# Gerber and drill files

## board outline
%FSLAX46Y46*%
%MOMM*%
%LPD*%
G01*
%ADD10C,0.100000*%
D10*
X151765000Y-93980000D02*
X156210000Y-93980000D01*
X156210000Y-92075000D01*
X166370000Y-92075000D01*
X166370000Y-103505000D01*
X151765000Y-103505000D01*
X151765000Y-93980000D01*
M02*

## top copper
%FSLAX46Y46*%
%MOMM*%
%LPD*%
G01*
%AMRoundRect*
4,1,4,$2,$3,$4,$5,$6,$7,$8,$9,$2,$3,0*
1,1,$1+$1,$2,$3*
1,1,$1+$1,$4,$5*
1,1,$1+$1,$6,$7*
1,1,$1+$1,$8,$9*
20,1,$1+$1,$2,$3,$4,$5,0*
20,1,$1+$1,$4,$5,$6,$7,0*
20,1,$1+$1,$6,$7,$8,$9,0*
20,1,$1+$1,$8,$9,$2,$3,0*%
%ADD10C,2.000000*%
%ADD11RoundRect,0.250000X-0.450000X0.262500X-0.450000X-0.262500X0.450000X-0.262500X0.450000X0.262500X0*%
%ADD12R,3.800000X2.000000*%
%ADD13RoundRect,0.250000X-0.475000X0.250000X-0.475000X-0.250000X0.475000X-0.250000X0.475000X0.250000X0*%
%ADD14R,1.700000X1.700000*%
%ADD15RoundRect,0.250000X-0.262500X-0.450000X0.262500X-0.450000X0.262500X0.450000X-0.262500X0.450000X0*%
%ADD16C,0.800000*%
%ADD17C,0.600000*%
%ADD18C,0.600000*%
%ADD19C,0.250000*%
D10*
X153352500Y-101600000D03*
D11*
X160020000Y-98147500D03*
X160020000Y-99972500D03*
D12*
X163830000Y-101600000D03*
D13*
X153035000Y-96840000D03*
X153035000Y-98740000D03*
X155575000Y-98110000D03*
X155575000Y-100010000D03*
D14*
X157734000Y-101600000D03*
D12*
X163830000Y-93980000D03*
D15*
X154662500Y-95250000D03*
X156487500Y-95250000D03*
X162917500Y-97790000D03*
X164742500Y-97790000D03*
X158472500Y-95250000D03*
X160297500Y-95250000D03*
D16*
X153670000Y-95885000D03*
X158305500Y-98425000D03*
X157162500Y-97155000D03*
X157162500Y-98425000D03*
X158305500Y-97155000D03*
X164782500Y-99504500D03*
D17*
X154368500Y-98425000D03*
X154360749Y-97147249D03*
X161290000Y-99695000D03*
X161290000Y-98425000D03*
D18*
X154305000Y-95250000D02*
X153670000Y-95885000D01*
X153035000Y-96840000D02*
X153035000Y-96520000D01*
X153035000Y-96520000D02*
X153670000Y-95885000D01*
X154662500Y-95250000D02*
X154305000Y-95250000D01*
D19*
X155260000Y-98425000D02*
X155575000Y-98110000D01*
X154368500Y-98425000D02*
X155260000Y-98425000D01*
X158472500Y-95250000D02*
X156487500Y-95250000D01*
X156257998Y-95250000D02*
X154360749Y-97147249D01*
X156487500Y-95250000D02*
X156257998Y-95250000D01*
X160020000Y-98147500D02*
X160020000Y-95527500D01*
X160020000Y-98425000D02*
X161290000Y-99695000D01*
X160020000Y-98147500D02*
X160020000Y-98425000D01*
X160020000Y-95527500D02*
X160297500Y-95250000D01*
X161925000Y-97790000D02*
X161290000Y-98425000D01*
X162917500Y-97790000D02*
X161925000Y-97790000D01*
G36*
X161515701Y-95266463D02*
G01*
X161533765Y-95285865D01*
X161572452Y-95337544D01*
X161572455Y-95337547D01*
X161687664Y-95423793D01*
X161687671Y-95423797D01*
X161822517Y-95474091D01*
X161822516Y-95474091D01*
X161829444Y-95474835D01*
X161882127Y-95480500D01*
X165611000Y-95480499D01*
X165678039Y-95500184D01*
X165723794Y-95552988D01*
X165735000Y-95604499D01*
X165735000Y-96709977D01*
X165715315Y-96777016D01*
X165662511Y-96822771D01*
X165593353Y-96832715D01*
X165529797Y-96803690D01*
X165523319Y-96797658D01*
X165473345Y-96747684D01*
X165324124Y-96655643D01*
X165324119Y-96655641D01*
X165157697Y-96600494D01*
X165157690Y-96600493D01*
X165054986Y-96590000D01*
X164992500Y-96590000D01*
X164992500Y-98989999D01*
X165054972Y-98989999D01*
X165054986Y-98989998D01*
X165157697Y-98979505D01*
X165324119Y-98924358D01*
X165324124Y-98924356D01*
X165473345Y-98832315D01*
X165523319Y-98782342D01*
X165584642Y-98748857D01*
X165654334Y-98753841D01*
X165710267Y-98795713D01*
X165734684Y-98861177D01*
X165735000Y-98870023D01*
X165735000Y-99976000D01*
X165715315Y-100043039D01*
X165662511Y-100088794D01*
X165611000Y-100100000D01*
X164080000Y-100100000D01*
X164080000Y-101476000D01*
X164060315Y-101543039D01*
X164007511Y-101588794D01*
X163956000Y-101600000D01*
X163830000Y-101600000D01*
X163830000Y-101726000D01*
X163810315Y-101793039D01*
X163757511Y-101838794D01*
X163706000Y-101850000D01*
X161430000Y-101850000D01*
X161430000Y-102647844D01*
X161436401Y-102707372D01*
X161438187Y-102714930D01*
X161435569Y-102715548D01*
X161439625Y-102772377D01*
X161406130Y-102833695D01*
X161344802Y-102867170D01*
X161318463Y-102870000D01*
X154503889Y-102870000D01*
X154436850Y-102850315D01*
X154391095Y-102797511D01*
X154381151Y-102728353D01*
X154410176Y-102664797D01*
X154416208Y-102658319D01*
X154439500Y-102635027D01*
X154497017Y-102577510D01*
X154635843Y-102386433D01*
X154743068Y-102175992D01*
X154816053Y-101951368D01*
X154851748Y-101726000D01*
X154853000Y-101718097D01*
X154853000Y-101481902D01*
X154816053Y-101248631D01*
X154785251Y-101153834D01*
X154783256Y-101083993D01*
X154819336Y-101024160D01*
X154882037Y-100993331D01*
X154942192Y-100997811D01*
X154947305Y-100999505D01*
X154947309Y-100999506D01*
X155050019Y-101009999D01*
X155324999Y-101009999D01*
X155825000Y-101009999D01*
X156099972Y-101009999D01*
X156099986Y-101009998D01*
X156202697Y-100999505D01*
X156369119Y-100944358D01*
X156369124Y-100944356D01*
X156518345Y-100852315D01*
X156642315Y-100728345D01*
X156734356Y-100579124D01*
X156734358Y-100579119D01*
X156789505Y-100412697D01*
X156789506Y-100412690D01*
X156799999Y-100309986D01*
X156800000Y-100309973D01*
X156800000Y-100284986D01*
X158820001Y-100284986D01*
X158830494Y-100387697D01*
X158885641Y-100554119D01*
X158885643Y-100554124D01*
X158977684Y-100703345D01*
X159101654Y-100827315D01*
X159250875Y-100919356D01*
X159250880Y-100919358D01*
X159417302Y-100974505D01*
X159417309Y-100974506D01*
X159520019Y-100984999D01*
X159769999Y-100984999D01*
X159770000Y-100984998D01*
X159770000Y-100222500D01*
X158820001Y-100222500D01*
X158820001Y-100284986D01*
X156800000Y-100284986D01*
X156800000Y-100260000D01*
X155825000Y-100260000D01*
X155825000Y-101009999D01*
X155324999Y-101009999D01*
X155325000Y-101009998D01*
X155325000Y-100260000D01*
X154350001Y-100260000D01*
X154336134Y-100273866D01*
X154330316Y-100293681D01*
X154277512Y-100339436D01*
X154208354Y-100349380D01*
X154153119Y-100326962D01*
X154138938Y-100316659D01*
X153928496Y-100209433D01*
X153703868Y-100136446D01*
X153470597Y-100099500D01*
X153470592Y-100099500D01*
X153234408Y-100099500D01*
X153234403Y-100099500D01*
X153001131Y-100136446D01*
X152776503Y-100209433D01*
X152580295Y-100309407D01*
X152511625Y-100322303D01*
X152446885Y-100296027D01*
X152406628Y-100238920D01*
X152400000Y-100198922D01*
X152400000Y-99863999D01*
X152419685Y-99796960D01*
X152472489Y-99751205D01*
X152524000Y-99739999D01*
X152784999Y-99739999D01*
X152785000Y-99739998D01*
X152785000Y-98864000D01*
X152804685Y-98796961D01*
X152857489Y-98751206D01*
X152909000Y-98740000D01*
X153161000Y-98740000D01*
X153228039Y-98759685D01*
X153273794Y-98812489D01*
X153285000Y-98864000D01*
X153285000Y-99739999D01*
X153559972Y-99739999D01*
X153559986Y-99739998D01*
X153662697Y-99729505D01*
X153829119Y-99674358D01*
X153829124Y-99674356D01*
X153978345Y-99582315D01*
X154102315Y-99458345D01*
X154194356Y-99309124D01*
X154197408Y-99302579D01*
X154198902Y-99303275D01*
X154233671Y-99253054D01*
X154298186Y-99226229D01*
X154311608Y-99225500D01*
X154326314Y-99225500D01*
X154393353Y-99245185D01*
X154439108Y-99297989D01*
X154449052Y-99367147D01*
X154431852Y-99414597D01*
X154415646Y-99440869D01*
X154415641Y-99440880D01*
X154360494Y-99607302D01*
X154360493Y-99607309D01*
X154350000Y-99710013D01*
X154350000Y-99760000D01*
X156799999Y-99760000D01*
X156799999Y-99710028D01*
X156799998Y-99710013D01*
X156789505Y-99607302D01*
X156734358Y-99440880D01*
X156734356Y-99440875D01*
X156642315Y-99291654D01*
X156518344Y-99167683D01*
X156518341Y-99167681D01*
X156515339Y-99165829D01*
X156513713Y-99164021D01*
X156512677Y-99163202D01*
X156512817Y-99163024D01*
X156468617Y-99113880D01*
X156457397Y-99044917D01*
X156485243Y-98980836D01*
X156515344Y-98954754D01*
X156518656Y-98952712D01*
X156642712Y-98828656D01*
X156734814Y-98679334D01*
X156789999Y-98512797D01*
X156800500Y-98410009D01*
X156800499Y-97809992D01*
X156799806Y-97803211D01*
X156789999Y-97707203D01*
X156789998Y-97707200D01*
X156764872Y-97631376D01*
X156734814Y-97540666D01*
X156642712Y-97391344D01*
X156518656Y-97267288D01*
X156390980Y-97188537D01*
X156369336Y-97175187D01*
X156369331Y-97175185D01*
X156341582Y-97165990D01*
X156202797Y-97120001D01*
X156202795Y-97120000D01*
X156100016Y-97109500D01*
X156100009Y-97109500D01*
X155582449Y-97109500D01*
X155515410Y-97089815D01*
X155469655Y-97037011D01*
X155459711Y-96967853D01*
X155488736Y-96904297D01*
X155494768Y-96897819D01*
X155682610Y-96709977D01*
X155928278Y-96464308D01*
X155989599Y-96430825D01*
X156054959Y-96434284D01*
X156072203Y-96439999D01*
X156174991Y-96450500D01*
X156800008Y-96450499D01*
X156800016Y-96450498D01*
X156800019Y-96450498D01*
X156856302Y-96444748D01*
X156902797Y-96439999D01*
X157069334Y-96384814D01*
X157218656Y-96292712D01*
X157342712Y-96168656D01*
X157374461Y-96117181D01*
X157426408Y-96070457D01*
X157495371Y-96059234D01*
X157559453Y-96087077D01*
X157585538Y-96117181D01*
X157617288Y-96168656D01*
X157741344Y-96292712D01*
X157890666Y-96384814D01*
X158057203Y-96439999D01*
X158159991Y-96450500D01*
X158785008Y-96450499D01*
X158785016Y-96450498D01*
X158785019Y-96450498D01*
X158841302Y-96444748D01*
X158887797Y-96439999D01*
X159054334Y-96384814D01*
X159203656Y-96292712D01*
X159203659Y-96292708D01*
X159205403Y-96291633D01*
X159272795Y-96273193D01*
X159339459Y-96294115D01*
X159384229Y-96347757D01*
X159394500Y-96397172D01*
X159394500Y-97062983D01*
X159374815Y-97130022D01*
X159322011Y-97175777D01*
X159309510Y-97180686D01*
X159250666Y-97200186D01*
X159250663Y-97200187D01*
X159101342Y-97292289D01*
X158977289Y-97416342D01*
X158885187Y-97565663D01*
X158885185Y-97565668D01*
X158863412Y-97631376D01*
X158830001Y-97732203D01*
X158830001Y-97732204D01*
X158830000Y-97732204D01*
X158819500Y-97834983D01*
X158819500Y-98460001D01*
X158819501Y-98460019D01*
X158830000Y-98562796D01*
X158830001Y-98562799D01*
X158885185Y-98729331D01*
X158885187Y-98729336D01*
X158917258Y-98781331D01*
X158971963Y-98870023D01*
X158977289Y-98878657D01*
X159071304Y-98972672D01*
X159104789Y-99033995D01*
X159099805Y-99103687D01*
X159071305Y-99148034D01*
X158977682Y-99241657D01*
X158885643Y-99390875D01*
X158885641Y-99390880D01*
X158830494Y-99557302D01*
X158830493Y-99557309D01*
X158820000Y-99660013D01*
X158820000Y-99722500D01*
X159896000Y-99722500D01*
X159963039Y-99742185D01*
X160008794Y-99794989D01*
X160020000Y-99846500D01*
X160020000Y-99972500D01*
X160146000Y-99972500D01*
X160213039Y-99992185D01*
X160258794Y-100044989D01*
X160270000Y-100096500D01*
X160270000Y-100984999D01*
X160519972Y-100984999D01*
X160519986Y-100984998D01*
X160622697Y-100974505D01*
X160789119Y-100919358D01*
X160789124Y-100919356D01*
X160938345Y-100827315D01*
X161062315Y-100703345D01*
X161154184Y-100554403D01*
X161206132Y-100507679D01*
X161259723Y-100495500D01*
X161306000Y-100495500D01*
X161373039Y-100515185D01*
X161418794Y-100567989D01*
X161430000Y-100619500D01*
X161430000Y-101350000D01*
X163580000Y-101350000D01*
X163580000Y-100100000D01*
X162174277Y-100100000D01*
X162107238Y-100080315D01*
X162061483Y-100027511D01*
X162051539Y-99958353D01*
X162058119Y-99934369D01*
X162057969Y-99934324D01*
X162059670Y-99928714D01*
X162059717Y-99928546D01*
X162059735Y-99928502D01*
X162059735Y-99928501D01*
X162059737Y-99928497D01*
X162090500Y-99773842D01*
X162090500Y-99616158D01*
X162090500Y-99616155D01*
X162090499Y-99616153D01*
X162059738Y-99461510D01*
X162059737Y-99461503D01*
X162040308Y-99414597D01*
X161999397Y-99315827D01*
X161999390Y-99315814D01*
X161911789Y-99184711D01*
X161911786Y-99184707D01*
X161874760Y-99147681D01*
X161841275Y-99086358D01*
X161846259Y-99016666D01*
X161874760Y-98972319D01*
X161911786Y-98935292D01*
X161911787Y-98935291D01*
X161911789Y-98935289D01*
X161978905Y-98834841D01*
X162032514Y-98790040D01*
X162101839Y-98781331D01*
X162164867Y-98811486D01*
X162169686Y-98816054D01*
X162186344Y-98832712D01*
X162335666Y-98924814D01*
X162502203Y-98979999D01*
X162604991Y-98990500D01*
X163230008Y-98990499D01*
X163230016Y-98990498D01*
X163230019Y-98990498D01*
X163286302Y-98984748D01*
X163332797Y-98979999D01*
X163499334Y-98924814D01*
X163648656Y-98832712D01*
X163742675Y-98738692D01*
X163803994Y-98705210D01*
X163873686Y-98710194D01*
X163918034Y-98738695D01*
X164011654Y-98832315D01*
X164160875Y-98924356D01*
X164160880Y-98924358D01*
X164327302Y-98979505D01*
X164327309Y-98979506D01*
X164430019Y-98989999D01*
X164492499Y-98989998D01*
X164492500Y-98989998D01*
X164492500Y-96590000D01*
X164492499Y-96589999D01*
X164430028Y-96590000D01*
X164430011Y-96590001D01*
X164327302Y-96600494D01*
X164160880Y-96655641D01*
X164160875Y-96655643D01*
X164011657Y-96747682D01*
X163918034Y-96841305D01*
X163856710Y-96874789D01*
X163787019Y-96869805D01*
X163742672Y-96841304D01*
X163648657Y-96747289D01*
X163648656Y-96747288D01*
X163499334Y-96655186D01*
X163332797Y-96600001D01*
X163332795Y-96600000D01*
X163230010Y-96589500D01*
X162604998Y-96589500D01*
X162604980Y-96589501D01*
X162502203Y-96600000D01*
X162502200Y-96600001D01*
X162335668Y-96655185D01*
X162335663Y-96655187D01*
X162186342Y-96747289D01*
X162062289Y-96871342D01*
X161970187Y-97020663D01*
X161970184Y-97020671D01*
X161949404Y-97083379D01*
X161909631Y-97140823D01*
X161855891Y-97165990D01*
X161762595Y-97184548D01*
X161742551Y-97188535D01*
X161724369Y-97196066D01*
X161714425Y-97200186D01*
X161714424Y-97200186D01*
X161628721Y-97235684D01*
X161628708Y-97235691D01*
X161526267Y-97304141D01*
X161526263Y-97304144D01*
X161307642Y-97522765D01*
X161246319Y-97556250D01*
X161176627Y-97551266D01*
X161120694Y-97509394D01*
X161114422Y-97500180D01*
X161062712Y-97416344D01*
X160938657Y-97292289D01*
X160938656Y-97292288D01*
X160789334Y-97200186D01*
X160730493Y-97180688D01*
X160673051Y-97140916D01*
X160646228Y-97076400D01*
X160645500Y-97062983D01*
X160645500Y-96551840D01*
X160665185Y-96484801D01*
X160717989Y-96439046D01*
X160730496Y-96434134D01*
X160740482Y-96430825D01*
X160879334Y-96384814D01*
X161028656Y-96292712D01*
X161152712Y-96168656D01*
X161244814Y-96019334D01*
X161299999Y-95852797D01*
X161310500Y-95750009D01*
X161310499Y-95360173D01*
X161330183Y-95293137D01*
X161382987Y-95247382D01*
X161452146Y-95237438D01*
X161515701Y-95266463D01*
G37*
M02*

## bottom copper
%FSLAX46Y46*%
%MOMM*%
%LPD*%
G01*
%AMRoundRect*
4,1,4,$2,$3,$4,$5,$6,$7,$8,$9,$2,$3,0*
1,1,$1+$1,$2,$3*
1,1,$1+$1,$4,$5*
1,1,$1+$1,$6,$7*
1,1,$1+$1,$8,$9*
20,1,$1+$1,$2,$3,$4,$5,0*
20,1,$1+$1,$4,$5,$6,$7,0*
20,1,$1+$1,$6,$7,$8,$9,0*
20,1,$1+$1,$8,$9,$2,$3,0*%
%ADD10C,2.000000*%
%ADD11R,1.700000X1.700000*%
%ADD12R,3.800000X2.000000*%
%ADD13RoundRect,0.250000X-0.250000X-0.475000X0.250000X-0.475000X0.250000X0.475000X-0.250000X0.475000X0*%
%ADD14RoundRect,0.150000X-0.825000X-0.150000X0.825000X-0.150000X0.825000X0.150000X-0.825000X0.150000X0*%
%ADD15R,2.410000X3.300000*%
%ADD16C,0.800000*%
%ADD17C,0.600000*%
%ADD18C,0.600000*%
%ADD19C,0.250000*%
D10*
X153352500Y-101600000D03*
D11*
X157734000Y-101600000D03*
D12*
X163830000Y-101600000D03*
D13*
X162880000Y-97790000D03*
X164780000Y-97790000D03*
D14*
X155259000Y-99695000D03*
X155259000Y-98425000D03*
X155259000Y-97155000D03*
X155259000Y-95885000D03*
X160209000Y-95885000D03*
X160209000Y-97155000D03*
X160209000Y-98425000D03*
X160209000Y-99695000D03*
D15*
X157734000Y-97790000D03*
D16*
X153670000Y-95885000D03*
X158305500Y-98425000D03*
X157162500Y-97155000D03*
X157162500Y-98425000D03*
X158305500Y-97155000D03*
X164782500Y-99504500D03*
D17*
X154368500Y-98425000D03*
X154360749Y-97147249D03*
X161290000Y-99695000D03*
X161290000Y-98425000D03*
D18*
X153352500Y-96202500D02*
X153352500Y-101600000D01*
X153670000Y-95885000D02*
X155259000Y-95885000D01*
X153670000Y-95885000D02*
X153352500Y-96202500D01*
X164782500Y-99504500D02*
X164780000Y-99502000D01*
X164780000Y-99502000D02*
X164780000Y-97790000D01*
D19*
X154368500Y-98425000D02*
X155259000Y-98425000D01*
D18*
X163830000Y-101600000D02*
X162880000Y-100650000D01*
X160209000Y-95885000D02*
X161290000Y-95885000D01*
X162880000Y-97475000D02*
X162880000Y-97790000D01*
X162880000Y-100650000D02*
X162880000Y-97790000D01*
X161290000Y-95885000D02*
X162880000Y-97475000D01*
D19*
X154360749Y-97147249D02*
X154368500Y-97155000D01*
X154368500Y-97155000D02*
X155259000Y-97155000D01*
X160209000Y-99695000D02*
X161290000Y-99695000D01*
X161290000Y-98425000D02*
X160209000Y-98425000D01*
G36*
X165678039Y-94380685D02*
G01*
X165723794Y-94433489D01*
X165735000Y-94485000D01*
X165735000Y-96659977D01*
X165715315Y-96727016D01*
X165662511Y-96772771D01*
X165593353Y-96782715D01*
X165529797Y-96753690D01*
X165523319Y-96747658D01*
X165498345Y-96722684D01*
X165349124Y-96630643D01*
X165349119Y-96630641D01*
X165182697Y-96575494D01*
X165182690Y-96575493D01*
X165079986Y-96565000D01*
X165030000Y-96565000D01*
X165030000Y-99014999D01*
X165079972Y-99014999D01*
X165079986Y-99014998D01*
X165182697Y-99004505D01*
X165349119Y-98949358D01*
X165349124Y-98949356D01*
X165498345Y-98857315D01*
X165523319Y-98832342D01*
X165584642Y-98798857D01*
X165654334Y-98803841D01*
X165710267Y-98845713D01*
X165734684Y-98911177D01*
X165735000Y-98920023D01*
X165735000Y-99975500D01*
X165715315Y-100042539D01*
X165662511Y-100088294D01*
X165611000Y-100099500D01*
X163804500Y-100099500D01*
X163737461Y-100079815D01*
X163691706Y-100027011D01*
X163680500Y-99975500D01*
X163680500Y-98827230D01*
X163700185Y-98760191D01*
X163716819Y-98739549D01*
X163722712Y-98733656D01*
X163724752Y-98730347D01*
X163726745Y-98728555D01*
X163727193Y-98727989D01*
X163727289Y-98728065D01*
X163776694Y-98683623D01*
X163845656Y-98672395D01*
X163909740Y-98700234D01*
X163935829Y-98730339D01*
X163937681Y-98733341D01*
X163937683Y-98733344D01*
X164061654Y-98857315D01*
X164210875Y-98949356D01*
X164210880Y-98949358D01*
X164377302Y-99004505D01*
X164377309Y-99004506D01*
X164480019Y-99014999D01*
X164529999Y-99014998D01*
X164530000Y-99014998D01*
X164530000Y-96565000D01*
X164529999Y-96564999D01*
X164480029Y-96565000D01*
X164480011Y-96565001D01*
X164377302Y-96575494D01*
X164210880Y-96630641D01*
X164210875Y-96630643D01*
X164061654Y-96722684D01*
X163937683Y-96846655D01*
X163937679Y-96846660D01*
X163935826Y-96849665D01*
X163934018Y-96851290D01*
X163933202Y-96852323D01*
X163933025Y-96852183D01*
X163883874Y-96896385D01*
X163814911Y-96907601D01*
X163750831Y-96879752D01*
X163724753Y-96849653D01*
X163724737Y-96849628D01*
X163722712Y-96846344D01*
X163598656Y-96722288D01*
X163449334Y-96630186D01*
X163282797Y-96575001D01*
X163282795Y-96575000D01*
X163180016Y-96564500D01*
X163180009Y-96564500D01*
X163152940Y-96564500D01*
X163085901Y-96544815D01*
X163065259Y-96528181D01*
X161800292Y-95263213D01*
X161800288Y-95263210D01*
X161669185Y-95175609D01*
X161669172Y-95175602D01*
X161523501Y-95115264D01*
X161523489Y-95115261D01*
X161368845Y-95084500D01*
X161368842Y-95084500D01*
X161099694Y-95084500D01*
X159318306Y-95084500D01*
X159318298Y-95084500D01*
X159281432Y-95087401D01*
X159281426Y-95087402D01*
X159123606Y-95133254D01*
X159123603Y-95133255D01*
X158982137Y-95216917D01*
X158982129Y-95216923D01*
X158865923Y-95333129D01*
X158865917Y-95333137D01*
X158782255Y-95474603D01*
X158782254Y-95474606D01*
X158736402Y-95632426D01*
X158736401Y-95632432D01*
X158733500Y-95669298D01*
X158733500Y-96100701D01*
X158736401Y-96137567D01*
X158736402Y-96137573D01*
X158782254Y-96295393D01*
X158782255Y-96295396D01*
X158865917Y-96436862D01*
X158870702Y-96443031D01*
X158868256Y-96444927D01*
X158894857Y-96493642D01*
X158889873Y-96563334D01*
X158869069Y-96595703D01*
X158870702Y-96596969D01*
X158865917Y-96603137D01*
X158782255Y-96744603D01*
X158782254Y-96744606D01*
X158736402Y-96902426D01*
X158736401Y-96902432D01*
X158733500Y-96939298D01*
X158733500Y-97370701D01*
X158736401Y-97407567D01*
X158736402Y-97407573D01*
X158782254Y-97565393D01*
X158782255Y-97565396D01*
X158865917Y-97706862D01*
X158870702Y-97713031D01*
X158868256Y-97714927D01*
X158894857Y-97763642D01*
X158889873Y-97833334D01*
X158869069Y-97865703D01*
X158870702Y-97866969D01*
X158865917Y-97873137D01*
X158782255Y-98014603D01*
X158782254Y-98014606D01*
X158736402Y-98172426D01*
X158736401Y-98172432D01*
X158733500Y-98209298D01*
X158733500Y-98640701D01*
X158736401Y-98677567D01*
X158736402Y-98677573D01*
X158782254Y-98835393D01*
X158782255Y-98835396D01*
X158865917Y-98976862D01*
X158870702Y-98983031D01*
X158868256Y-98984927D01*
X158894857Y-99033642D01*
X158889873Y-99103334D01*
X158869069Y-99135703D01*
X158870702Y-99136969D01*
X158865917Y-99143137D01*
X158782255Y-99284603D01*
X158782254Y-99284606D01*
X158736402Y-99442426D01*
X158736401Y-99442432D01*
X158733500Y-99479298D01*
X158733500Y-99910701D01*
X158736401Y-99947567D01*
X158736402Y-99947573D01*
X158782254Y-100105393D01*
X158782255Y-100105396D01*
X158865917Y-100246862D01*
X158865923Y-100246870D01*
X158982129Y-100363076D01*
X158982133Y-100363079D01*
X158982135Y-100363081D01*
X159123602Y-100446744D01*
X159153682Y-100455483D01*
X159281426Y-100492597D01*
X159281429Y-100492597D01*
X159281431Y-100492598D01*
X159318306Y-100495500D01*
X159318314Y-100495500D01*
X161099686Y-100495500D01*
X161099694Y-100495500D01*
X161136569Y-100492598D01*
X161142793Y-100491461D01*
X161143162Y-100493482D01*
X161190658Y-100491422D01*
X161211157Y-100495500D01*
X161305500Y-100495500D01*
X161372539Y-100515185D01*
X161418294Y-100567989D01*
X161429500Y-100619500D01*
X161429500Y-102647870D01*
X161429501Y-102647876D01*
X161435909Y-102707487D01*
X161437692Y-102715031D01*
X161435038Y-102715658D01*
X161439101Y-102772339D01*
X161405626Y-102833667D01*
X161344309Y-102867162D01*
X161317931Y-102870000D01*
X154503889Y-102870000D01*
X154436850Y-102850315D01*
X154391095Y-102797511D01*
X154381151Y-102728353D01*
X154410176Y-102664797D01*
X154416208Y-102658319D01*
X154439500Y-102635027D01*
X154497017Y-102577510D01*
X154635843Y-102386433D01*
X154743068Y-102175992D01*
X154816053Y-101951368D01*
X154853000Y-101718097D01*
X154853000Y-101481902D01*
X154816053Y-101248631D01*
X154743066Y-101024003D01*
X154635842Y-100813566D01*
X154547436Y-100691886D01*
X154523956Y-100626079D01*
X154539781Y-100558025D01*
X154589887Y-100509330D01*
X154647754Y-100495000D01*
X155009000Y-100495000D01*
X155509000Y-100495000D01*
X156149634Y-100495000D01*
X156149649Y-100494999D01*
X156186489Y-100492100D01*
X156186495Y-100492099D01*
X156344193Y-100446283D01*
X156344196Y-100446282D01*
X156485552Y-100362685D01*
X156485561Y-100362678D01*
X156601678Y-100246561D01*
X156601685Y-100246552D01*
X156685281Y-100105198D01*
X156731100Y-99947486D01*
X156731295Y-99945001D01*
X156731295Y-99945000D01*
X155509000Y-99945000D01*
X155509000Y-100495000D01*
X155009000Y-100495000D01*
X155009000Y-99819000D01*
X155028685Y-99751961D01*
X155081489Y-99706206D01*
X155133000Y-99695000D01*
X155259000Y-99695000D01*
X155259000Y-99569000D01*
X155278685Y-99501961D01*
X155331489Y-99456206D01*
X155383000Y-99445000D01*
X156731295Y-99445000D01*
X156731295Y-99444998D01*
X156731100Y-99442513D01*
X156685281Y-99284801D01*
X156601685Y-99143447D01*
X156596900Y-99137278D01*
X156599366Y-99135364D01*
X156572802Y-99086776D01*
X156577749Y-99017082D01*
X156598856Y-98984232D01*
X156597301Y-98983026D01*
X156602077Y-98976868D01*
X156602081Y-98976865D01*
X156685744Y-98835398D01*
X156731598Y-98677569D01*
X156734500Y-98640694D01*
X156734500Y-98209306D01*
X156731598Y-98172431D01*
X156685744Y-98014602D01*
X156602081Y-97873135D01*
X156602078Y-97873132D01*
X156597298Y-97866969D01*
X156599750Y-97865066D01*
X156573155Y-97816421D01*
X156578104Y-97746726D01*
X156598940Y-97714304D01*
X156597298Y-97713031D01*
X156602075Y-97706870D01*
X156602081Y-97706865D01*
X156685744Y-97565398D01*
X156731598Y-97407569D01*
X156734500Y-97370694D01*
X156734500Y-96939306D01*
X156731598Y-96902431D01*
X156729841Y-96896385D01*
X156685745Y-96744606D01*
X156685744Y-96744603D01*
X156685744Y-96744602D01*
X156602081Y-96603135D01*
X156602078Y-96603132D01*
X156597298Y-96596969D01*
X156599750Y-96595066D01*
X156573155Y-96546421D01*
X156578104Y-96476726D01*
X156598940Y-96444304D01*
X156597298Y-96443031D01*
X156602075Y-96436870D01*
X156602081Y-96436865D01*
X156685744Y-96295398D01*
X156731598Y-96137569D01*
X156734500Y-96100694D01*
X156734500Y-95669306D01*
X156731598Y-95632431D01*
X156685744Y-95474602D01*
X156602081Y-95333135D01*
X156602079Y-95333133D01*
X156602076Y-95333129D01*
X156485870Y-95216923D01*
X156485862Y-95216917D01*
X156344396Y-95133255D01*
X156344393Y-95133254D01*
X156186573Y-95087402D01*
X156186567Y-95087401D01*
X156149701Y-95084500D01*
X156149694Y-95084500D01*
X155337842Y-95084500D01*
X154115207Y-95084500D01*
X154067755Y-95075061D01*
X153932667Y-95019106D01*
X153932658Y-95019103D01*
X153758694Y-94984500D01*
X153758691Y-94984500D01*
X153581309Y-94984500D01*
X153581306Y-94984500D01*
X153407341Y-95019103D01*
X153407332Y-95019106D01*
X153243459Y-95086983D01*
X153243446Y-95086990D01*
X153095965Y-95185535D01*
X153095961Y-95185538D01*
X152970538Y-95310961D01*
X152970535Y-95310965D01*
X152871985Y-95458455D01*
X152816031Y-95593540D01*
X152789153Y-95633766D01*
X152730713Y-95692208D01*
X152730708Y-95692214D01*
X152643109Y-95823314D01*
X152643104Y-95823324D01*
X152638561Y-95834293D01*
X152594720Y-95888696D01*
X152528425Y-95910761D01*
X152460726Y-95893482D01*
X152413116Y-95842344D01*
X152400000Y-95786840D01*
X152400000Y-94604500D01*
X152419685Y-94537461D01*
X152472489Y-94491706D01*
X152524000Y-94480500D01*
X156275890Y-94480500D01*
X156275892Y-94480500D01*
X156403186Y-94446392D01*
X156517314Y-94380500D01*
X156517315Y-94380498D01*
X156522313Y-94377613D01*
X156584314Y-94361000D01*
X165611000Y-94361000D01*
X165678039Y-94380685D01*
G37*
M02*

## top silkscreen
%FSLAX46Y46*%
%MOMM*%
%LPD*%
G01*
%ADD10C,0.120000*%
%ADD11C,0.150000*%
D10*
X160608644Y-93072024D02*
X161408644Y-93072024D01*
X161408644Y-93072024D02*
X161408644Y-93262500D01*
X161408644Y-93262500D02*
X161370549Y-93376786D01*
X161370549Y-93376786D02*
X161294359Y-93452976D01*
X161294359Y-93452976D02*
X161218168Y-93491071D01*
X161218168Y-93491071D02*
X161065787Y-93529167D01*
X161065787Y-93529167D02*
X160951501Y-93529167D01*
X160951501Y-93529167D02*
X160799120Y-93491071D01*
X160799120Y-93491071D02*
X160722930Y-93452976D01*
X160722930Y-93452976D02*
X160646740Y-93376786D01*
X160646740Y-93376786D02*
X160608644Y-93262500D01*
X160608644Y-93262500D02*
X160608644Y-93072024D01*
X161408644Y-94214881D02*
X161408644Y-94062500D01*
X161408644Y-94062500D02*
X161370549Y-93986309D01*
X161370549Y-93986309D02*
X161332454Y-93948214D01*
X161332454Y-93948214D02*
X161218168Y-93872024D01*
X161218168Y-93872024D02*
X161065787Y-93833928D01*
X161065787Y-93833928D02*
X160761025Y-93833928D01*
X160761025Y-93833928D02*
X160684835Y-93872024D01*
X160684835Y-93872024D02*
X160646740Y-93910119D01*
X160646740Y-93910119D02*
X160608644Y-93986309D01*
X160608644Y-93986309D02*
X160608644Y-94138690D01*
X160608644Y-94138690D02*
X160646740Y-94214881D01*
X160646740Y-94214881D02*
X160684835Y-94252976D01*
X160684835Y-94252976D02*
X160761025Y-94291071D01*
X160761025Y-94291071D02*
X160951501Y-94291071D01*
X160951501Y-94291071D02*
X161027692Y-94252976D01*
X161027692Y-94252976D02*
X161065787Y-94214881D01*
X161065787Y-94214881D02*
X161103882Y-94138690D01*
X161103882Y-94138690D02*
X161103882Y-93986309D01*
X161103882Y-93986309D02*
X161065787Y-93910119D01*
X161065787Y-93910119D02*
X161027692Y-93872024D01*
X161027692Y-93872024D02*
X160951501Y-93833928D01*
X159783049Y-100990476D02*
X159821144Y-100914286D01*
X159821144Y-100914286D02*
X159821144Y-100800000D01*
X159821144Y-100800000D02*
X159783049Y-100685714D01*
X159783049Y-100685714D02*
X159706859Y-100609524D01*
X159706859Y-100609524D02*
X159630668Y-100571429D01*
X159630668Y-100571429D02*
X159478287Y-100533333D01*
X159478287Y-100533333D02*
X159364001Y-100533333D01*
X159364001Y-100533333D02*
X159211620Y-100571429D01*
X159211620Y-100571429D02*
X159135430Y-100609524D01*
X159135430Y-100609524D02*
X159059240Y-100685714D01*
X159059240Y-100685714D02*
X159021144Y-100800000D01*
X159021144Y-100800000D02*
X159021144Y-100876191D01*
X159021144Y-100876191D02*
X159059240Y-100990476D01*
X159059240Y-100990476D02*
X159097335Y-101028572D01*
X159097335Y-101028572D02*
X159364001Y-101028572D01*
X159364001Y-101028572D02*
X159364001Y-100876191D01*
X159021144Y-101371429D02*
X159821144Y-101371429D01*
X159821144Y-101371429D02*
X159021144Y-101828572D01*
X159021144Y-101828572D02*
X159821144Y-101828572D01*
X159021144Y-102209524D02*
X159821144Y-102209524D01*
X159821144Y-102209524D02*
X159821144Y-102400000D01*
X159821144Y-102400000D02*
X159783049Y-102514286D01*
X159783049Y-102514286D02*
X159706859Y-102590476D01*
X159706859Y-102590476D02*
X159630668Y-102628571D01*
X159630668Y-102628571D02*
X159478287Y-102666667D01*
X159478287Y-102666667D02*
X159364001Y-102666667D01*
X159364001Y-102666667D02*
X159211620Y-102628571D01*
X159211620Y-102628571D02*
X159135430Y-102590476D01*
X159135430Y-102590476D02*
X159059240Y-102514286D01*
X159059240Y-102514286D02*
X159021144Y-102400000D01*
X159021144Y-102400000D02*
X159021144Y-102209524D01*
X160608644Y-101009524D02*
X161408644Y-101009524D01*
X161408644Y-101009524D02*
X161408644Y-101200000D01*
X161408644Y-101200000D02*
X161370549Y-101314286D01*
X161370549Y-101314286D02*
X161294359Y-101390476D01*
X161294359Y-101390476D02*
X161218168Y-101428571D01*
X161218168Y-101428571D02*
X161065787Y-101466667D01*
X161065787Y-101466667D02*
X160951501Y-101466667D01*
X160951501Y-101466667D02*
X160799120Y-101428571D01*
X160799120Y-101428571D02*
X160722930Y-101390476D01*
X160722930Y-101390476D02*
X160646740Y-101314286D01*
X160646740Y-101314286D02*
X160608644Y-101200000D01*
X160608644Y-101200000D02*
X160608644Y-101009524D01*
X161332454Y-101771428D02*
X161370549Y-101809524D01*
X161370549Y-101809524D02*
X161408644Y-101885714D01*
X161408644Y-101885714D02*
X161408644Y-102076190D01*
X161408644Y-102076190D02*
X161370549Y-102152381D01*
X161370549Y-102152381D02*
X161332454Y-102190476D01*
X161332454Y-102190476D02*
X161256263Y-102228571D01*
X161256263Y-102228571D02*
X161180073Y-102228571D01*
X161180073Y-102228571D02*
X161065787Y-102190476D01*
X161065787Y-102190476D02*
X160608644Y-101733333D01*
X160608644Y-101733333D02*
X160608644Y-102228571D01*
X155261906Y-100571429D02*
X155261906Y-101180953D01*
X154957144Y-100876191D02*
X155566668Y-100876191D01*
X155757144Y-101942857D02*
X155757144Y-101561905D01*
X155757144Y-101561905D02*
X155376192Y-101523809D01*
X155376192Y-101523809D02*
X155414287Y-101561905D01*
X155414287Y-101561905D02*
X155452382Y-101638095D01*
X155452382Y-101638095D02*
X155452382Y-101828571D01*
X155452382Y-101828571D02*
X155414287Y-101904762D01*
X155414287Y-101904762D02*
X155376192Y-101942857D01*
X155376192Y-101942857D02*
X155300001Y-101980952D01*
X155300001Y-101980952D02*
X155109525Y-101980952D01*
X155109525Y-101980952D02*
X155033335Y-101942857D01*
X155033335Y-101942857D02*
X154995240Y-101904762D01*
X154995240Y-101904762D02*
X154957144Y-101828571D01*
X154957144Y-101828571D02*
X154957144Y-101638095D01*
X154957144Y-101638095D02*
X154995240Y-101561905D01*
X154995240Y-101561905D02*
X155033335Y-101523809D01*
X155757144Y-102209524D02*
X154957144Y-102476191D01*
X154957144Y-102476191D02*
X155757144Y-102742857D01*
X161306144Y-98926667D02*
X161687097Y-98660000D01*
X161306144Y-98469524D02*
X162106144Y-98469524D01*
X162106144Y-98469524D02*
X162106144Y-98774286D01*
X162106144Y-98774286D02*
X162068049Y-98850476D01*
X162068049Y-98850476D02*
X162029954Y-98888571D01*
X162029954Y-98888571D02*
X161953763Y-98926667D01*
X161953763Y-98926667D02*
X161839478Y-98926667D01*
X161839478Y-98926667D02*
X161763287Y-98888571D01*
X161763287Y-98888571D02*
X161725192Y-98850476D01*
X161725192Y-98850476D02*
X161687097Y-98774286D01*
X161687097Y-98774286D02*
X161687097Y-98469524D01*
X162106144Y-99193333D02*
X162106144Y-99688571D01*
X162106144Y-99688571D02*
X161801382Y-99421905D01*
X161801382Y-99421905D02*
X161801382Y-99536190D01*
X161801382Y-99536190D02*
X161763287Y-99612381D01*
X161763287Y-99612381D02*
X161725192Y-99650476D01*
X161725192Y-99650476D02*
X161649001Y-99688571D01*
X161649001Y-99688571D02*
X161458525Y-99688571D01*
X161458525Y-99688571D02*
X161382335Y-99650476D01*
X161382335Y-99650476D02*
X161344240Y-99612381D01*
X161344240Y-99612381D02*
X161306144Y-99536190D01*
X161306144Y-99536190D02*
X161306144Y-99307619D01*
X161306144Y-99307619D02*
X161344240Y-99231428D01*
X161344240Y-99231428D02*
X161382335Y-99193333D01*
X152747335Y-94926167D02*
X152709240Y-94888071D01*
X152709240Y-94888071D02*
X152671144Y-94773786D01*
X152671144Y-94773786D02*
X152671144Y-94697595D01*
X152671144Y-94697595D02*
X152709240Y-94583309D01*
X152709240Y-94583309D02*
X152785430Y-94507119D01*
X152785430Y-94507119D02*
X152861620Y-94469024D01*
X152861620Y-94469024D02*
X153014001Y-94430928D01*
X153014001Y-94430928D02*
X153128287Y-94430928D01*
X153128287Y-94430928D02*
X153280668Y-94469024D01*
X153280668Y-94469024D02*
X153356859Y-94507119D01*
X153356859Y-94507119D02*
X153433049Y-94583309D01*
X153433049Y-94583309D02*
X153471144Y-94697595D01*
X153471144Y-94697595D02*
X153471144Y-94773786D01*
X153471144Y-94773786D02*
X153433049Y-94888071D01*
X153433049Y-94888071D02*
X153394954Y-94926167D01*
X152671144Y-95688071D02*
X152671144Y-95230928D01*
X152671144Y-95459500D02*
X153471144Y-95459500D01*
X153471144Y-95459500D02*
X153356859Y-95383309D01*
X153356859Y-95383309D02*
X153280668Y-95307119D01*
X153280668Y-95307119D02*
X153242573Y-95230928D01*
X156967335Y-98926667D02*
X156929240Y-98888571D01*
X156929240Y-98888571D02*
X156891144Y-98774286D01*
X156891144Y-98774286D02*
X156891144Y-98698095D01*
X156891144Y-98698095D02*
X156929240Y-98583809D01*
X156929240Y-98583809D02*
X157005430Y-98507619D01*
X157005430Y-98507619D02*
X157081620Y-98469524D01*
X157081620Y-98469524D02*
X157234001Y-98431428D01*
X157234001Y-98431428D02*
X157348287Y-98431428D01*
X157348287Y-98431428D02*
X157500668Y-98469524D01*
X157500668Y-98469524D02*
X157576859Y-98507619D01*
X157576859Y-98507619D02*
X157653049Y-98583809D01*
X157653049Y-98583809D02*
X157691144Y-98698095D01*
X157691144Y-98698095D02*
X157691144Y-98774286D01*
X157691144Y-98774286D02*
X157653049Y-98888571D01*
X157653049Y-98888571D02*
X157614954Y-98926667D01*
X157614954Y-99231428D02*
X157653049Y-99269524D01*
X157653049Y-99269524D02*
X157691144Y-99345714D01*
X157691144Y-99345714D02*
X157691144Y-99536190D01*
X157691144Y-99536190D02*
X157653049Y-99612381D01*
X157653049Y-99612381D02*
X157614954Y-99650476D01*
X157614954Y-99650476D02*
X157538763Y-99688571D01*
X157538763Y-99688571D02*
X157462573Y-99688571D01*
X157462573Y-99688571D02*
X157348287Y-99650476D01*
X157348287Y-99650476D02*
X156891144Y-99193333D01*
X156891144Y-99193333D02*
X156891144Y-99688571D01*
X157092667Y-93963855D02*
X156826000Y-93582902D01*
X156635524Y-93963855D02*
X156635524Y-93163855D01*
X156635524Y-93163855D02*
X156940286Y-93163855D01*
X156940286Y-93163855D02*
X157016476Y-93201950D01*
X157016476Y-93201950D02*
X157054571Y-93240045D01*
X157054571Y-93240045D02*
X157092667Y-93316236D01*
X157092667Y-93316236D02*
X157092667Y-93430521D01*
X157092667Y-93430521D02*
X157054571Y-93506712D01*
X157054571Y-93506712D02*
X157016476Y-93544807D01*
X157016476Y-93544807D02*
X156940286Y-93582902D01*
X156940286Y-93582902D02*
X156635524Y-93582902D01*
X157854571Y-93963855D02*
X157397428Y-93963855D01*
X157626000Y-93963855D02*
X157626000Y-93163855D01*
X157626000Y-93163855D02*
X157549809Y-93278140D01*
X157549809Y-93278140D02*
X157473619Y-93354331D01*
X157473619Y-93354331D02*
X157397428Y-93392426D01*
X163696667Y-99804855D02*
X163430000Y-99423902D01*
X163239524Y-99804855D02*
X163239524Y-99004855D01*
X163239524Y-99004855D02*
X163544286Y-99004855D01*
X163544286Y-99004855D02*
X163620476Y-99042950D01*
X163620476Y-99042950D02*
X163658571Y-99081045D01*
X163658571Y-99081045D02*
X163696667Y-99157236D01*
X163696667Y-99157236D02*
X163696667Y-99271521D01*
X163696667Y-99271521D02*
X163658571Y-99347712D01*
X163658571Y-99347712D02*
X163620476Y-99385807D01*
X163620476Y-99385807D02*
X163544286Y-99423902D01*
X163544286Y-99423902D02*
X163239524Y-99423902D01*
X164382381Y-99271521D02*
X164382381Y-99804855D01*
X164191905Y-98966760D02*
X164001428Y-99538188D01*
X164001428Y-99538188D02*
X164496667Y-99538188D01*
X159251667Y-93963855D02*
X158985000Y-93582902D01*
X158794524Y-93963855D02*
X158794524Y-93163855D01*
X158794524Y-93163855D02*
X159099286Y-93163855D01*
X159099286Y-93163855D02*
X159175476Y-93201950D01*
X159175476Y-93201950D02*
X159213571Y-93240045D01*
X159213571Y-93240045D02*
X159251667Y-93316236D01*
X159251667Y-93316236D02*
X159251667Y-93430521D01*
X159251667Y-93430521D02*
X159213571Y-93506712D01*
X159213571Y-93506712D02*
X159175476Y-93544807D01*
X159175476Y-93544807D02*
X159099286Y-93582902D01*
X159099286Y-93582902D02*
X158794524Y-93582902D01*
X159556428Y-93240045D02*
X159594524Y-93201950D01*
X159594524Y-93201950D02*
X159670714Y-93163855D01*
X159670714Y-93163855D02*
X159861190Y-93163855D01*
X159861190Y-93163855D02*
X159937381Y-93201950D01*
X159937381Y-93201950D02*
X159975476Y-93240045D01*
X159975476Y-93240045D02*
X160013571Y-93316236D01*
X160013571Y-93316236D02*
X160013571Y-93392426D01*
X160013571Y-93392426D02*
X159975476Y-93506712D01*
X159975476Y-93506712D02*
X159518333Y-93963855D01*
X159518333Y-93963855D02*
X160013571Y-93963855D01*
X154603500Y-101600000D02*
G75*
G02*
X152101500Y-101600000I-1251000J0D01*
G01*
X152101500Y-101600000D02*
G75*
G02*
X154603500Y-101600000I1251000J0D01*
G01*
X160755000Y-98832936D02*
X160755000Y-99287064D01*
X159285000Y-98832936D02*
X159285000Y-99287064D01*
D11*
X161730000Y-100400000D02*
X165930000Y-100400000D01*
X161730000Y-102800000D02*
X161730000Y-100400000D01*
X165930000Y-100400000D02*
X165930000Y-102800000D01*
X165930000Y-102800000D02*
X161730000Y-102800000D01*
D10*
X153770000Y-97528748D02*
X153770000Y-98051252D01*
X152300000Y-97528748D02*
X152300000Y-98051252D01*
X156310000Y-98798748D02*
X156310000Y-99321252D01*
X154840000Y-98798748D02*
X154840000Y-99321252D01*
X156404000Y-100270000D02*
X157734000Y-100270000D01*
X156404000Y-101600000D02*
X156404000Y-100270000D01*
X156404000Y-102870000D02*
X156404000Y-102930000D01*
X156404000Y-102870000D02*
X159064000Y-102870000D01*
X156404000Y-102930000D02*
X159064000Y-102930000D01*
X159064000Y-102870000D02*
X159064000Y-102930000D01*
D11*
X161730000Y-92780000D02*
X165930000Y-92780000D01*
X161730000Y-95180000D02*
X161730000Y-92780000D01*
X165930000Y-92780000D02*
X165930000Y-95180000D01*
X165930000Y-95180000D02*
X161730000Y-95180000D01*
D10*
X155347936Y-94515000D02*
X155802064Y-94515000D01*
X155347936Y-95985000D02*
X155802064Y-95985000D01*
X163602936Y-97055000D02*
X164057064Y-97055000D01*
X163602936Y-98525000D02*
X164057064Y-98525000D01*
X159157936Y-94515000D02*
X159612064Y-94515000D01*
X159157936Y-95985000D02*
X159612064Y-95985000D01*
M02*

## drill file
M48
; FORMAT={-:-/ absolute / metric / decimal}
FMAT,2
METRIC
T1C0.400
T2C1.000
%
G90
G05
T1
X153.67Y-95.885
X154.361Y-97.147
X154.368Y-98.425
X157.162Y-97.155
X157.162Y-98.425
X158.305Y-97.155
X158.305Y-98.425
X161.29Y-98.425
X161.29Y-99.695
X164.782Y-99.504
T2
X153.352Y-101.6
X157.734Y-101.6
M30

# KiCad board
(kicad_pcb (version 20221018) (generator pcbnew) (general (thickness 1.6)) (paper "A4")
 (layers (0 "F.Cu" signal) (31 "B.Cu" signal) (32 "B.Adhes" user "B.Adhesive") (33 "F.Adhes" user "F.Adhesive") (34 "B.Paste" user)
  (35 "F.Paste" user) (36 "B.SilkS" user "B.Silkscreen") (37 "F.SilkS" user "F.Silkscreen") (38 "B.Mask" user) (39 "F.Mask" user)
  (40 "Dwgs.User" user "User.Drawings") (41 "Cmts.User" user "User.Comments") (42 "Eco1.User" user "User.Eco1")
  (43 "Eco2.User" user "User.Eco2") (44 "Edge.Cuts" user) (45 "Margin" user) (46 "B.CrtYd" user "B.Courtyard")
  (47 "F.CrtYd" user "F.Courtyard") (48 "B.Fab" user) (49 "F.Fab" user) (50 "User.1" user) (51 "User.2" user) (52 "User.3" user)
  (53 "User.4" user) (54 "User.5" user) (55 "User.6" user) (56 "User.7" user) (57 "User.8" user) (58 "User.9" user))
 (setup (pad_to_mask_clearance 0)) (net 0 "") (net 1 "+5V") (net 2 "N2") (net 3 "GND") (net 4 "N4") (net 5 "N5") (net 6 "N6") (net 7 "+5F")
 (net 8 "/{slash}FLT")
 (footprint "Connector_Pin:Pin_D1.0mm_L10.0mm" (layer "F.Cu") (at 153.3525 101.6)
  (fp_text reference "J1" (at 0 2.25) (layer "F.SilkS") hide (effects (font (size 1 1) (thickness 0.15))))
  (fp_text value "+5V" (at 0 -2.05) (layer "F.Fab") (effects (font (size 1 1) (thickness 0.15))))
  (fp_circle (center 0 0) (end 1.25 0.05) (stroke (width 0.12) (type solid)) (fill none) (layer "F.SilkS"))
  (pad "1" thru_hole circle (at 0 0) (size 2 2) (drill 1) (layers "*.Cu" "*.Mask") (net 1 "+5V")))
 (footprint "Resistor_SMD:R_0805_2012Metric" (layer "F.Cu") (at 160.02 99.06 -90)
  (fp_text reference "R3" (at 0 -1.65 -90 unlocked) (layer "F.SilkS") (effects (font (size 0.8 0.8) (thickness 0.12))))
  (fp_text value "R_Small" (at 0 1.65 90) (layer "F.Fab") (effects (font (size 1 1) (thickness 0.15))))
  (fp_line (start -0.227064 -0.735) (end 0.227064 -0.735) (stroke (width 0.12) (type solid)) (layer "F.SilkS"))
  (fp_line (start -0.227064 0.735) (end 0.227064 0.735) (stroke (width 0.12) (type solid)) (layer "F.SilkS"))
  (pad "1" smd roundrect (at -0.9125 0 270) (size 1.025 1.4) (layers "F.Cu" "F.Paste" "F.Mask") (roundrect_rratio 0.243902) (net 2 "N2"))
  (pad "2" smd roundrect (at 0.9125 0 270) (size 1.025 1.4) (layers "F.Cu" "F.Paste" "F.Mask") (roundrect_rratio 0.243902) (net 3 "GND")))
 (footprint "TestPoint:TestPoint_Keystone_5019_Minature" (layer "F.Cu") (at 163.83 101.6)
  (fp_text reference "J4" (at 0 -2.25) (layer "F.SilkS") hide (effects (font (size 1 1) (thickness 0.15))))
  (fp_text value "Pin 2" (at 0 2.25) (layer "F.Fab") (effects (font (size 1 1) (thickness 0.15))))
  (fp_line (start -2.1 -1.2) (end 2.1 -1.2) (stroke (width 0.15) (type solid)) (layer "F.SilkS"))
  (fp_line (start -2.1 1.2) (end -2.1 -1.2) (stroke (width 0.15) (type solid)) (layer "F.SilkS"))
  (fp_line (start 2.1 -1.2) (end 2.1 1.2) (stroke (width 0.15) (type solid)) (layer "F.SilkS"))
  (fp_line (start 2.1 1.2) (end -2.1 1.2) (stroke (width 0.15) (type solid)) (layer "F.SilkS"))
  (pad "1" smd rect (at 0 0) (size 3.8 2) (layers "F.Cu" "F.Paste" "F.Mask") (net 3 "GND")))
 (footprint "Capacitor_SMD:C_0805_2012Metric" (layer "F.Cu") (at 153.035 97.79 -90)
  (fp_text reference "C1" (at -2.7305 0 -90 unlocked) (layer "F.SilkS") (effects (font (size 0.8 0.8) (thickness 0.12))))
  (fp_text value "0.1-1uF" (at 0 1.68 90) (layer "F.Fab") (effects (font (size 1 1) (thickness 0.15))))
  (fp_line (start -0.261252 -0.735) (end 0.261252 -0.735) (stroke (width 0.12) (type solid)) (layer "F.SilkS"))
  (fp_line (start -0.261252 0.735) (end 0.261252 0.735) (stroke (width 0.12) (type solid)) (layer "F.SilkS"))
  (pad "1" smd roundrect (at -0.95 0 270) (size 1 1.45) (layers "F.Cu" "F.Paste" "F.Mask") (roundrect_rratio 0.25) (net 1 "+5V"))
  (pad "2" smd roundrect (at 0.95 0 270) (size 1 1.45) (layers "F.Cu" "F.Paste" "F.Mask") (roundrect_rratio 0.25) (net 3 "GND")))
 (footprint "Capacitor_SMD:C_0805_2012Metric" (layer "F.Cu") (at 155.575 99.06 -90)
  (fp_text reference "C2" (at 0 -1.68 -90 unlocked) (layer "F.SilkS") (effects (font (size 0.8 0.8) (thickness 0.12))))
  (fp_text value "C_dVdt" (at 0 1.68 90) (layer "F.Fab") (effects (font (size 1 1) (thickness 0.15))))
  (fp_line (start -0.261252 -0.735) (end 0.261252 -0.735) (stroke (width 0.12) (type solid)) (layer "F.SilkS"))
  (fp_line (start -0.261252 0.735) (end 0.261252 0.735) (stroke (width 0.12) (type solid)) (layer "F.SilkS"))
  (pad "1" smd roundrect (at -0.95 0 270) (size 1 1.45) (layers "F.Cu" "F.Paste" "F.Mask") (roundrect_rratio 0.25) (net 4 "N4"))
  (pad "2" smd roundrect (at 0.95 0 270) (size 1 1.45) (layers "F.Cu" "F.Paste" "F.Mask") (roundrect_rratio 0.25) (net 3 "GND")))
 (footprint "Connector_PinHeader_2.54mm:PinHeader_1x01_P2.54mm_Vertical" (layer "F.Cu") (at 157.734 101.6)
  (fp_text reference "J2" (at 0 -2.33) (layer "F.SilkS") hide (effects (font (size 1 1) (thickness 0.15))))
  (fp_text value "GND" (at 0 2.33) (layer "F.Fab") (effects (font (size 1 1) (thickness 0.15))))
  (fp_line (start -1.33 -1.33) (end 0 -1.33) (stroke (width 0.12) (type solid)) (layer "F.SilkS"))
  (fp_line (start -1.33 0) (end -1.33 -1.33) (stroke (width 0.12) (type solid)) (layer "F.SilkS"))
  (fp_line (start -1.33 1.27) (end -1.33 1.33) (stroke (width 0.12) (type solid)) (layer "F.SilkS"))
  (fp_line (start -1.33 1.27) (end 1.33 1.27) (stroke (width 0.12) (type solid)) (layer "F.SilkS"))
  (fp_line (start -1.33 1.33) (end 1.33 1.33) (stroke (width 0.12) (type solid)) (layer "F.SilkS"))
  (fp_line (start 1.33 1.27) (end 1.33 1.33) (stroke (width 0.12) (type solid)) (layer "F.SilkS"))
  (pad "1" thru_hole rect (at 0 0) (size 1.7 1.7) (drill 1) (layers "*.Cu" "*.Mask") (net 3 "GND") (zone_connect 2)))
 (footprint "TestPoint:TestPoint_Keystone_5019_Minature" (layer "F.Cu") (at 163.83 93.98)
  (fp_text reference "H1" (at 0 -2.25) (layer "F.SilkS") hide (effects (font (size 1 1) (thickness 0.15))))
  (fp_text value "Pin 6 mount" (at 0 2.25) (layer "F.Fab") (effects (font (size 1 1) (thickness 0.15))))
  (fp_line (start -2.1 -1.2) (end 2.1 -1.2) (stroke (width 0.15) (type solid)) (layer "F.SilkS"))
  (fp_line (start -2.1 1.2) (end -2.1 -1.2) (stroke (width 0.15) (type solid)) (layer "F.SilkS"))
  (fp_line (start 2.1 -1.2) (end 2.1 1.2) (stroke (width 0.15) (type solid)) (layer "F.SilkS"))
  (fp_line (start 2.1 1.2) (end -2.1 1.2) (stroke (width 0.15) (type solid)) (layer "F.SilkS"))
  (pad "1" smd rect (at 0 0) (size 3.8 2) (layers "F.Cu" "F.Paste" "F.Mask")))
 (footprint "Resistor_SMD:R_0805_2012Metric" (layer "F.Cu") (at 155.575 95.25)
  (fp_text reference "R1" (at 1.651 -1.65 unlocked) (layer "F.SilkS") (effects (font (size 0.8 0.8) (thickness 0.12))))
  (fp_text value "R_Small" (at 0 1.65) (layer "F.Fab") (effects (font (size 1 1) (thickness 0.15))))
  (fp_line (start -0.227064 -0.735) (end 0.227064 -0.735) (stroke (width 0.12) (type solid)) (layer "F.SilkS"))
  (fp_line (start -0.227064 0.735) (end 0.227064 0.735) (stroke (width 0.12) (type solid)) (layer "F.SilkS"))
  (pad "1" smd roundrect (at -0.9125 0) (size 1.025 1.4) (layers "F.Cu" "F.Paste" "F.Mask") (roundrect_rratio 0.243902) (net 1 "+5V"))
  (pad "2" smd roundrect (at 0.9125 0) (size 1.025 1.4) (layers "F.Cu" "F.Paste" "F.Mask") (roundrect_rratio 0.243902) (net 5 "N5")))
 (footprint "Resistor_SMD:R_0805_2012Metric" (layer "F.Cu") (at 163.83 97.79)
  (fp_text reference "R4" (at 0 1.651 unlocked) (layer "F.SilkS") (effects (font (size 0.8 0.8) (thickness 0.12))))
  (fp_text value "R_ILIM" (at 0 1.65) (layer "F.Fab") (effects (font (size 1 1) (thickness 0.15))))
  (fp_line (start -0.227064 -0.735) (end 0.227064 -0.735) (stroke (width 0.12) (type solid)) (layer "F.SilkS"))
  (fp_line (start -0.227064 0.735) (end 0.227064 0.735) (stroke (width 0.12) (type solid)) (layer "F.SilkS"))
  (pad "1" smd roundrect (at -0.9125 0) (size 1.025 1.4) (layers "F.Cu" "F.Paste" "F.Mask") (roundrect_rratio 0.243902) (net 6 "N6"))
  (pad "2" smd roundrect (at 0.9125 0) (size 1.025 1.4) (layers "F.Cu" "F.Paste" "F.Mask") (roundrect_rratio 0.243902) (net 3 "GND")))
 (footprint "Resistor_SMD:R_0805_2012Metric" (layer "F.Cu") (at 159.385 95.25)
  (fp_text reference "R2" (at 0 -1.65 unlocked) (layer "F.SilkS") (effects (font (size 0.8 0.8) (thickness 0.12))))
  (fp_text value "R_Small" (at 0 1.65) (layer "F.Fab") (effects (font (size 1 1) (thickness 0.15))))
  (fp_line (start -0.227064 -0.735) (end 0.227064 -0.735) (stroke (width 0.12) (type solid)) (layer "F.SilkS"))
  (fp_line (start -0.227064 0.735) (end 0.227064 0.735) (stroke (width 0.12) (type solid)) (layer "F.SilkS"))
  (pad "1" smd roundrect (at -0.9125 0) (size 1.025 1.4) (layers "F.Cu" "F.Paste" "F.Mask") (roundrect_rratio 0.243902) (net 5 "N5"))
  (pad "2" smd roundrect (at 0.9125 0) (size 1.025 1.4) (layers "F.Cu" "F.Paste" "F.Mask") (roundrect_rratio 0.243902) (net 2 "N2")))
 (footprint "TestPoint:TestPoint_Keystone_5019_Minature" (layer "B.Cu") (at 163.83 101.6 180)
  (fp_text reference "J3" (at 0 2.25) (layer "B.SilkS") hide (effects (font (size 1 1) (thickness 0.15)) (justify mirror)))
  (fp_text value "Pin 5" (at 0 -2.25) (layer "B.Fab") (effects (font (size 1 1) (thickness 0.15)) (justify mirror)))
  (pad "1" smd rect (at 0 0 180) (size 3.8 2) (layers "B.Cu" "B.Paste" "B.Mask") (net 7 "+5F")))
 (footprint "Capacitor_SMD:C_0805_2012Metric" (layer "B.Cu") (at 163.83 97.79)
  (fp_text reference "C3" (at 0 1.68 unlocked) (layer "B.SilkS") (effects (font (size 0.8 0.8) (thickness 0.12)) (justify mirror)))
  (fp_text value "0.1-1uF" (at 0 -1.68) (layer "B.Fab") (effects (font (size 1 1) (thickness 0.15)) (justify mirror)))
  (pad "1" smd roundrect (at -0.95 0) (size 1 1.45) (layers "B.Cu" "B.Paste" "B.Mask") (roundrect_rratio 0.25) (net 7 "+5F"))
  (pad "2" smd roundrect (at 0.95 0) (size 1 1.45) (layers "B.Cu" "B.Paste" "B.Mask") (roundrect_rratio 0.25) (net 3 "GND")))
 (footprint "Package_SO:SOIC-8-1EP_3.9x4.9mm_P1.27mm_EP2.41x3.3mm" (layer "B.Cu") (at 157.734 97.79)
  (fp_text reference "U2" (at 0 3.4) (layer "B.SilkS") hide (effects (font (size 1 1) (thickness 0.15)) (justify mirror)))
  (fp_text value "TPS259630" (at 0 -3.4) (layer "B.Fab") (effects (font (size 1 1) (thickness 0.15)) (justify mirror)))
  (pad "" smd roundrect (at -0.6 -0.825) (size 0.97 1.33) (layers "B.Paste") (roundrect_rratio 0.25))
  (pad "" smd roundrect (at -0.6 0.825) (size 0.97 1.33) (layers "B.Paste") (roundrect_rratio 0.25))
  (pad "" smd roundrect (at 0.6 -0.825) (size 0.97 1.33) (layers "B.Paste") (roundrect_rratio 0.25))
  (pad "" smd roundrect (at 0.6 0.825) (size 0.97 1.33) (layers "B.Paste") (roundrect_rratio 0.25))
  (pad "1" smd roundrect (at -2.475 1.905) (size 1.95 0.6) (layers "B.Cu" "B.Paste" "B.Mask") (roundrect_rratio 0.25) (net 3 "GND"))
  (pad "2" smd roundrect (at -2.475 0.635) (size 1.95 0.6) (layers "B.Cu" "B.Paste" "B.Mask") (roundrect_rratio 0.25) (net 4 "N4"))
  (pad "3" smd roundrect (at -2.475 -0.635) (size 1.95 0.6) (layers "B.Cu" "B.Paste" "B.Mask") (roundrect_rratio 0.25) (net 5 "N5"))
  (pad "4" smd roundrect (at -2.475 -1.905) (size 1.95 0.6) (layers "B.Cu" "B.Paste" "B.Mask") (roundrect_rratio 0.25) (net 1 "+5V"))
  (pad "5" smd roundrect (at 2.475 -1.905) (size 1.95 0.6) (layers "B.Cu" "B.Paste" "B.Mask") (roundrect_rratio 0.25) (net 7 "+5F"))
  (pad "6" smd roundrect (at 2.475 -0.635) (size 1.95 0.6) (layers "B.Cu" "B.Paste" "B.Mask") (roundrect_rratio 0.25) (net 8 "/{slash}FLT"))
  (pad "7" smd roundrect (at 2.475 0.635) (size 1.95 0.6) (layers "B.Cu" "B.Paste" "B.Mask") (roundrect_rratio 0.25) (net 6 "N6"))
  (pad "8" smd roundrect (at 2.475 1.905) (size 1.95 0.6) (layers "B.Cu" "B.Paste" "B.Mask") (roundrect_rratio 0.25) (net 2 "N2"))
  (pad "9" smd rect (at 0 0) (size 2.41 3.3) (layers "B.Cu" "B.Mask") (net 3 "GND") (zone_connect 2)))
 (gr_poly
  (pts (xy 151.765 93.98) (xy 156.21 93.98) (xy 156.21 92.075) (xy 166.37 92.075) (xy 166.37 103.505) (xy 151.765 103.505))
  (stroke (width 0.1) (type solid)) (fill none) (layer "Edge.Cuts"))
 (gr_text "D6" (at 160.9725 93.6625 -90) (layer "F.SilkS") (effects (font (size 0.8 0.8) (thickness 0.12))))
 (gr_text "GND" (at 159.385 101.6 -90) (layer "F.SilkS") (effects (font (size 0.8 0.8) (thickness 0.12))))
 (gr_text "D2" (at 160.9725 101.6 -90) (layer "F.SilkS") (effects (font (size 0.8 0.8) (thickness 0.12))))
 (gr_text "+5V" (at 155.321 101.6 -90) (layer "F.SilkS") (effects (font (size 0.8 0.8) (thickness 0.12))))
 (segment (start 154.305 95.25) (end 153.67 95.885) (width 0.6) (layer "F.Cu") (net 1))
 (segment (start 153.035 96.84) (end 153.035 96.52) (width 0.6) (layer "F.Cu") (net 1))
 (segment (start 153.035 96.52) (end 153.67 95.885) (width 0.6) (layer "F.Cu") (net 1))
 (segment (start 154.6625 95.25) (end 154.305 95.25) (width 0.6) (layer "F.Cu") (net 1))
 (via (at 153.67 95.885) (size 0.8) (drill 0.4) (layers "F.Cu" "B.Cu") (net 1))
 (segment (start 153.3525 96.2025) (end 153.3525 101.6) (width 0.6) (layer "B.Cu") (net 1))
 (segment (start 153.67 95.885) (end 155.259 95.885) (width 0.6) (layer "B.Cu") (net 1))
 (segment (start 153.67 95.885) (end 153.3525 96.2025) (width 0.6) (layer "B.Cu") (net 1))
 (via (at 158.3055 98.425) (size 0.8) (drill 0.4) (layers "F.Cu" "B.Cu") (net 3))
 (via (at 157.1625 97.155) (size 0.8) (drill 0.4) (layers "F.Cu" "B.Cu") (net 3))
 (via (at 157.1625 98.425) (size 0.8) (drill 0.4) (layers "F.Cu" "B.Cu") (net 3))
 (via (at 158.3055 97.155) (size 0.8) (drill 0.4) (layers "F.Cu" "B.Cu") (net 3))
 (via (at 164.7825 99.5045) (size 0.8) (drill 0.4) (layers "F.Cu" "B.Cu") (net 3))
 (segment (start 164.7825 99.5045) (end 164.78 99.502) (width 0.6) (layer "B.Cu") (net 3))
 (segment (start 164.78 99.502) (end 164.78 97.79) (width 0.6) (layer "B.Cu") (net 3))
 (segment (start 155.26 98.425) (end 155.575 98.11) (width 0.25) (layer "F.Cu") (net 4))
 (segment (start 154.3685 98.425) (end 155.26 98.425) (width 0.25) (layer "F.Cu") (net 4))
 (via (at 154.3685 98.425) (size 0.6) (drill 0.4) (layers "F.Cu" "B.Cu") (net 4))
 (segment (start 154.3685 98.425) (end 155.259 98.425) (width 0.25) (layer "B.Cu") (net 4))
 (segment (start 163.83 101.6) (end 162.88 100.65) (width 0.6) (layer "B.Cu") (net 7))
 (segment (start 160.209 95.885) (end 161.29 95.885) (width 0.6) (layer "B.Cu") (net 7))
 (segment (start 162.88 97.475) (end 162.88 97.79) (width 0.6) (layer "B.Cu") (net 7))
 (segment (start 162.88 100.65) (end 162.88 97.79) (width 0.6) (layer "B.Cu") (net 7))
 (segment (start 161.29 95.885) (end 162.88 97.475) (width 0.6) (layer "B.Cu") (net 7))
 (segment (start 158.4725 95.25) (end 156.4875 95.25) (width 0.25) (layer "F.Cu") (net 5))
 (segment (start 156.257998 95.25) (end 154.360749 97.147249) (width 0.25) (layer "F.Cu") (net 5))
 (segment (start 156.4875 95.25) (end 156.257998 95.25) (width 0.25) (layer "F.Cu") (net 5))
 (via (at 154.360749 97.147249) (size 0.6) (drill 0.4) (layers "F.Cu" "B.Cu") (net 5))
 (segment (start 154.360749 97.147249) (end 154.3685 97.155) (width 0.25) (layer "B.Cu") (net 5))
 (segment (start 154.3685 97.155) (end 155.259 97.155) (width 0.25) (layer "B.Cu") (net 5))
 (segment (start 160.02 98.1475) (end 160.02 95.5275) (width 0.25) (layer "F.Cu") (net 2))
 (segment (start 160.02 98.425) (end 161.29 99.695) (width 0.25) (layer "F.Cu") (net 2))
 (segment (start 160.02 98.1475) (end 160.02 98.425) (width 0.25) (layer "F.Cu") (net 2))
 (segment (start 160.02 95.5275) (end 160.2975 95.25) (width 0.25) (layer "F.Cu") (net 2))
 (via (at 161.29 99.695) (size 0.6) (drill 0.4) (layers "F.Cu" "B.Cu") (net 2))
 (segment (start 160.209 99.695) (end 161.29 99.695) (width 0.25) (layer "B.Cu") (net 2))
 (segment (start 161.925 97.79) (end 161.29 98.425) (width 0.25) (layer "F.Cu") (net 6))
 (segment (start 162.9175 97.79) (end 161.925 97.79) (width 0.25) (layer "F.Cu") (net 6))
 (via (at 161.29 98.425) (size 0.6) (drill 0.4) (layers "F.Cu" "B.Cu") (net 6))
 (segment (start 161.29 98.425) (end 160.209 98.425) (width 0.25) (layer "B.Cu") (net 6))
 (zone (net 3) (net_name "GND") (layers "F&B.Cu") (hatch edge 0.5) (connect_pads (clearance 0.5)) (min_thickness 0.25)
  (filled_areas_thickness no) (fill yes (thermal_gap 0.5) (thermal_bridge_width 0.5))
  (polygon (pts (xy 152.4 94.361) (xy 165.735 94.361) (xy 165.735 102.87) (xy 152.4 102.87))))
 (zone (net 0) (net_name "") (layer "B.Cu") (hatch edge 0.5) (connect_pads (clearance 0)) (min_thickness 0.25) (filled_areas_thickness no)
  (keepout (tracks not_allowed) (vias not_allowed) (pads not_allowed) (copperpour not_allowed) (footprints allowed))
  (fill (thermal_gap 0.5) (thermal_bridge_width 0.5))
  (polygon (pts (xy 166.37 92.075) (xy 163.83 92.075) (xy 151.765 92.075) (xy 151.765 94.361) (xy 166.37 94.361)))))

